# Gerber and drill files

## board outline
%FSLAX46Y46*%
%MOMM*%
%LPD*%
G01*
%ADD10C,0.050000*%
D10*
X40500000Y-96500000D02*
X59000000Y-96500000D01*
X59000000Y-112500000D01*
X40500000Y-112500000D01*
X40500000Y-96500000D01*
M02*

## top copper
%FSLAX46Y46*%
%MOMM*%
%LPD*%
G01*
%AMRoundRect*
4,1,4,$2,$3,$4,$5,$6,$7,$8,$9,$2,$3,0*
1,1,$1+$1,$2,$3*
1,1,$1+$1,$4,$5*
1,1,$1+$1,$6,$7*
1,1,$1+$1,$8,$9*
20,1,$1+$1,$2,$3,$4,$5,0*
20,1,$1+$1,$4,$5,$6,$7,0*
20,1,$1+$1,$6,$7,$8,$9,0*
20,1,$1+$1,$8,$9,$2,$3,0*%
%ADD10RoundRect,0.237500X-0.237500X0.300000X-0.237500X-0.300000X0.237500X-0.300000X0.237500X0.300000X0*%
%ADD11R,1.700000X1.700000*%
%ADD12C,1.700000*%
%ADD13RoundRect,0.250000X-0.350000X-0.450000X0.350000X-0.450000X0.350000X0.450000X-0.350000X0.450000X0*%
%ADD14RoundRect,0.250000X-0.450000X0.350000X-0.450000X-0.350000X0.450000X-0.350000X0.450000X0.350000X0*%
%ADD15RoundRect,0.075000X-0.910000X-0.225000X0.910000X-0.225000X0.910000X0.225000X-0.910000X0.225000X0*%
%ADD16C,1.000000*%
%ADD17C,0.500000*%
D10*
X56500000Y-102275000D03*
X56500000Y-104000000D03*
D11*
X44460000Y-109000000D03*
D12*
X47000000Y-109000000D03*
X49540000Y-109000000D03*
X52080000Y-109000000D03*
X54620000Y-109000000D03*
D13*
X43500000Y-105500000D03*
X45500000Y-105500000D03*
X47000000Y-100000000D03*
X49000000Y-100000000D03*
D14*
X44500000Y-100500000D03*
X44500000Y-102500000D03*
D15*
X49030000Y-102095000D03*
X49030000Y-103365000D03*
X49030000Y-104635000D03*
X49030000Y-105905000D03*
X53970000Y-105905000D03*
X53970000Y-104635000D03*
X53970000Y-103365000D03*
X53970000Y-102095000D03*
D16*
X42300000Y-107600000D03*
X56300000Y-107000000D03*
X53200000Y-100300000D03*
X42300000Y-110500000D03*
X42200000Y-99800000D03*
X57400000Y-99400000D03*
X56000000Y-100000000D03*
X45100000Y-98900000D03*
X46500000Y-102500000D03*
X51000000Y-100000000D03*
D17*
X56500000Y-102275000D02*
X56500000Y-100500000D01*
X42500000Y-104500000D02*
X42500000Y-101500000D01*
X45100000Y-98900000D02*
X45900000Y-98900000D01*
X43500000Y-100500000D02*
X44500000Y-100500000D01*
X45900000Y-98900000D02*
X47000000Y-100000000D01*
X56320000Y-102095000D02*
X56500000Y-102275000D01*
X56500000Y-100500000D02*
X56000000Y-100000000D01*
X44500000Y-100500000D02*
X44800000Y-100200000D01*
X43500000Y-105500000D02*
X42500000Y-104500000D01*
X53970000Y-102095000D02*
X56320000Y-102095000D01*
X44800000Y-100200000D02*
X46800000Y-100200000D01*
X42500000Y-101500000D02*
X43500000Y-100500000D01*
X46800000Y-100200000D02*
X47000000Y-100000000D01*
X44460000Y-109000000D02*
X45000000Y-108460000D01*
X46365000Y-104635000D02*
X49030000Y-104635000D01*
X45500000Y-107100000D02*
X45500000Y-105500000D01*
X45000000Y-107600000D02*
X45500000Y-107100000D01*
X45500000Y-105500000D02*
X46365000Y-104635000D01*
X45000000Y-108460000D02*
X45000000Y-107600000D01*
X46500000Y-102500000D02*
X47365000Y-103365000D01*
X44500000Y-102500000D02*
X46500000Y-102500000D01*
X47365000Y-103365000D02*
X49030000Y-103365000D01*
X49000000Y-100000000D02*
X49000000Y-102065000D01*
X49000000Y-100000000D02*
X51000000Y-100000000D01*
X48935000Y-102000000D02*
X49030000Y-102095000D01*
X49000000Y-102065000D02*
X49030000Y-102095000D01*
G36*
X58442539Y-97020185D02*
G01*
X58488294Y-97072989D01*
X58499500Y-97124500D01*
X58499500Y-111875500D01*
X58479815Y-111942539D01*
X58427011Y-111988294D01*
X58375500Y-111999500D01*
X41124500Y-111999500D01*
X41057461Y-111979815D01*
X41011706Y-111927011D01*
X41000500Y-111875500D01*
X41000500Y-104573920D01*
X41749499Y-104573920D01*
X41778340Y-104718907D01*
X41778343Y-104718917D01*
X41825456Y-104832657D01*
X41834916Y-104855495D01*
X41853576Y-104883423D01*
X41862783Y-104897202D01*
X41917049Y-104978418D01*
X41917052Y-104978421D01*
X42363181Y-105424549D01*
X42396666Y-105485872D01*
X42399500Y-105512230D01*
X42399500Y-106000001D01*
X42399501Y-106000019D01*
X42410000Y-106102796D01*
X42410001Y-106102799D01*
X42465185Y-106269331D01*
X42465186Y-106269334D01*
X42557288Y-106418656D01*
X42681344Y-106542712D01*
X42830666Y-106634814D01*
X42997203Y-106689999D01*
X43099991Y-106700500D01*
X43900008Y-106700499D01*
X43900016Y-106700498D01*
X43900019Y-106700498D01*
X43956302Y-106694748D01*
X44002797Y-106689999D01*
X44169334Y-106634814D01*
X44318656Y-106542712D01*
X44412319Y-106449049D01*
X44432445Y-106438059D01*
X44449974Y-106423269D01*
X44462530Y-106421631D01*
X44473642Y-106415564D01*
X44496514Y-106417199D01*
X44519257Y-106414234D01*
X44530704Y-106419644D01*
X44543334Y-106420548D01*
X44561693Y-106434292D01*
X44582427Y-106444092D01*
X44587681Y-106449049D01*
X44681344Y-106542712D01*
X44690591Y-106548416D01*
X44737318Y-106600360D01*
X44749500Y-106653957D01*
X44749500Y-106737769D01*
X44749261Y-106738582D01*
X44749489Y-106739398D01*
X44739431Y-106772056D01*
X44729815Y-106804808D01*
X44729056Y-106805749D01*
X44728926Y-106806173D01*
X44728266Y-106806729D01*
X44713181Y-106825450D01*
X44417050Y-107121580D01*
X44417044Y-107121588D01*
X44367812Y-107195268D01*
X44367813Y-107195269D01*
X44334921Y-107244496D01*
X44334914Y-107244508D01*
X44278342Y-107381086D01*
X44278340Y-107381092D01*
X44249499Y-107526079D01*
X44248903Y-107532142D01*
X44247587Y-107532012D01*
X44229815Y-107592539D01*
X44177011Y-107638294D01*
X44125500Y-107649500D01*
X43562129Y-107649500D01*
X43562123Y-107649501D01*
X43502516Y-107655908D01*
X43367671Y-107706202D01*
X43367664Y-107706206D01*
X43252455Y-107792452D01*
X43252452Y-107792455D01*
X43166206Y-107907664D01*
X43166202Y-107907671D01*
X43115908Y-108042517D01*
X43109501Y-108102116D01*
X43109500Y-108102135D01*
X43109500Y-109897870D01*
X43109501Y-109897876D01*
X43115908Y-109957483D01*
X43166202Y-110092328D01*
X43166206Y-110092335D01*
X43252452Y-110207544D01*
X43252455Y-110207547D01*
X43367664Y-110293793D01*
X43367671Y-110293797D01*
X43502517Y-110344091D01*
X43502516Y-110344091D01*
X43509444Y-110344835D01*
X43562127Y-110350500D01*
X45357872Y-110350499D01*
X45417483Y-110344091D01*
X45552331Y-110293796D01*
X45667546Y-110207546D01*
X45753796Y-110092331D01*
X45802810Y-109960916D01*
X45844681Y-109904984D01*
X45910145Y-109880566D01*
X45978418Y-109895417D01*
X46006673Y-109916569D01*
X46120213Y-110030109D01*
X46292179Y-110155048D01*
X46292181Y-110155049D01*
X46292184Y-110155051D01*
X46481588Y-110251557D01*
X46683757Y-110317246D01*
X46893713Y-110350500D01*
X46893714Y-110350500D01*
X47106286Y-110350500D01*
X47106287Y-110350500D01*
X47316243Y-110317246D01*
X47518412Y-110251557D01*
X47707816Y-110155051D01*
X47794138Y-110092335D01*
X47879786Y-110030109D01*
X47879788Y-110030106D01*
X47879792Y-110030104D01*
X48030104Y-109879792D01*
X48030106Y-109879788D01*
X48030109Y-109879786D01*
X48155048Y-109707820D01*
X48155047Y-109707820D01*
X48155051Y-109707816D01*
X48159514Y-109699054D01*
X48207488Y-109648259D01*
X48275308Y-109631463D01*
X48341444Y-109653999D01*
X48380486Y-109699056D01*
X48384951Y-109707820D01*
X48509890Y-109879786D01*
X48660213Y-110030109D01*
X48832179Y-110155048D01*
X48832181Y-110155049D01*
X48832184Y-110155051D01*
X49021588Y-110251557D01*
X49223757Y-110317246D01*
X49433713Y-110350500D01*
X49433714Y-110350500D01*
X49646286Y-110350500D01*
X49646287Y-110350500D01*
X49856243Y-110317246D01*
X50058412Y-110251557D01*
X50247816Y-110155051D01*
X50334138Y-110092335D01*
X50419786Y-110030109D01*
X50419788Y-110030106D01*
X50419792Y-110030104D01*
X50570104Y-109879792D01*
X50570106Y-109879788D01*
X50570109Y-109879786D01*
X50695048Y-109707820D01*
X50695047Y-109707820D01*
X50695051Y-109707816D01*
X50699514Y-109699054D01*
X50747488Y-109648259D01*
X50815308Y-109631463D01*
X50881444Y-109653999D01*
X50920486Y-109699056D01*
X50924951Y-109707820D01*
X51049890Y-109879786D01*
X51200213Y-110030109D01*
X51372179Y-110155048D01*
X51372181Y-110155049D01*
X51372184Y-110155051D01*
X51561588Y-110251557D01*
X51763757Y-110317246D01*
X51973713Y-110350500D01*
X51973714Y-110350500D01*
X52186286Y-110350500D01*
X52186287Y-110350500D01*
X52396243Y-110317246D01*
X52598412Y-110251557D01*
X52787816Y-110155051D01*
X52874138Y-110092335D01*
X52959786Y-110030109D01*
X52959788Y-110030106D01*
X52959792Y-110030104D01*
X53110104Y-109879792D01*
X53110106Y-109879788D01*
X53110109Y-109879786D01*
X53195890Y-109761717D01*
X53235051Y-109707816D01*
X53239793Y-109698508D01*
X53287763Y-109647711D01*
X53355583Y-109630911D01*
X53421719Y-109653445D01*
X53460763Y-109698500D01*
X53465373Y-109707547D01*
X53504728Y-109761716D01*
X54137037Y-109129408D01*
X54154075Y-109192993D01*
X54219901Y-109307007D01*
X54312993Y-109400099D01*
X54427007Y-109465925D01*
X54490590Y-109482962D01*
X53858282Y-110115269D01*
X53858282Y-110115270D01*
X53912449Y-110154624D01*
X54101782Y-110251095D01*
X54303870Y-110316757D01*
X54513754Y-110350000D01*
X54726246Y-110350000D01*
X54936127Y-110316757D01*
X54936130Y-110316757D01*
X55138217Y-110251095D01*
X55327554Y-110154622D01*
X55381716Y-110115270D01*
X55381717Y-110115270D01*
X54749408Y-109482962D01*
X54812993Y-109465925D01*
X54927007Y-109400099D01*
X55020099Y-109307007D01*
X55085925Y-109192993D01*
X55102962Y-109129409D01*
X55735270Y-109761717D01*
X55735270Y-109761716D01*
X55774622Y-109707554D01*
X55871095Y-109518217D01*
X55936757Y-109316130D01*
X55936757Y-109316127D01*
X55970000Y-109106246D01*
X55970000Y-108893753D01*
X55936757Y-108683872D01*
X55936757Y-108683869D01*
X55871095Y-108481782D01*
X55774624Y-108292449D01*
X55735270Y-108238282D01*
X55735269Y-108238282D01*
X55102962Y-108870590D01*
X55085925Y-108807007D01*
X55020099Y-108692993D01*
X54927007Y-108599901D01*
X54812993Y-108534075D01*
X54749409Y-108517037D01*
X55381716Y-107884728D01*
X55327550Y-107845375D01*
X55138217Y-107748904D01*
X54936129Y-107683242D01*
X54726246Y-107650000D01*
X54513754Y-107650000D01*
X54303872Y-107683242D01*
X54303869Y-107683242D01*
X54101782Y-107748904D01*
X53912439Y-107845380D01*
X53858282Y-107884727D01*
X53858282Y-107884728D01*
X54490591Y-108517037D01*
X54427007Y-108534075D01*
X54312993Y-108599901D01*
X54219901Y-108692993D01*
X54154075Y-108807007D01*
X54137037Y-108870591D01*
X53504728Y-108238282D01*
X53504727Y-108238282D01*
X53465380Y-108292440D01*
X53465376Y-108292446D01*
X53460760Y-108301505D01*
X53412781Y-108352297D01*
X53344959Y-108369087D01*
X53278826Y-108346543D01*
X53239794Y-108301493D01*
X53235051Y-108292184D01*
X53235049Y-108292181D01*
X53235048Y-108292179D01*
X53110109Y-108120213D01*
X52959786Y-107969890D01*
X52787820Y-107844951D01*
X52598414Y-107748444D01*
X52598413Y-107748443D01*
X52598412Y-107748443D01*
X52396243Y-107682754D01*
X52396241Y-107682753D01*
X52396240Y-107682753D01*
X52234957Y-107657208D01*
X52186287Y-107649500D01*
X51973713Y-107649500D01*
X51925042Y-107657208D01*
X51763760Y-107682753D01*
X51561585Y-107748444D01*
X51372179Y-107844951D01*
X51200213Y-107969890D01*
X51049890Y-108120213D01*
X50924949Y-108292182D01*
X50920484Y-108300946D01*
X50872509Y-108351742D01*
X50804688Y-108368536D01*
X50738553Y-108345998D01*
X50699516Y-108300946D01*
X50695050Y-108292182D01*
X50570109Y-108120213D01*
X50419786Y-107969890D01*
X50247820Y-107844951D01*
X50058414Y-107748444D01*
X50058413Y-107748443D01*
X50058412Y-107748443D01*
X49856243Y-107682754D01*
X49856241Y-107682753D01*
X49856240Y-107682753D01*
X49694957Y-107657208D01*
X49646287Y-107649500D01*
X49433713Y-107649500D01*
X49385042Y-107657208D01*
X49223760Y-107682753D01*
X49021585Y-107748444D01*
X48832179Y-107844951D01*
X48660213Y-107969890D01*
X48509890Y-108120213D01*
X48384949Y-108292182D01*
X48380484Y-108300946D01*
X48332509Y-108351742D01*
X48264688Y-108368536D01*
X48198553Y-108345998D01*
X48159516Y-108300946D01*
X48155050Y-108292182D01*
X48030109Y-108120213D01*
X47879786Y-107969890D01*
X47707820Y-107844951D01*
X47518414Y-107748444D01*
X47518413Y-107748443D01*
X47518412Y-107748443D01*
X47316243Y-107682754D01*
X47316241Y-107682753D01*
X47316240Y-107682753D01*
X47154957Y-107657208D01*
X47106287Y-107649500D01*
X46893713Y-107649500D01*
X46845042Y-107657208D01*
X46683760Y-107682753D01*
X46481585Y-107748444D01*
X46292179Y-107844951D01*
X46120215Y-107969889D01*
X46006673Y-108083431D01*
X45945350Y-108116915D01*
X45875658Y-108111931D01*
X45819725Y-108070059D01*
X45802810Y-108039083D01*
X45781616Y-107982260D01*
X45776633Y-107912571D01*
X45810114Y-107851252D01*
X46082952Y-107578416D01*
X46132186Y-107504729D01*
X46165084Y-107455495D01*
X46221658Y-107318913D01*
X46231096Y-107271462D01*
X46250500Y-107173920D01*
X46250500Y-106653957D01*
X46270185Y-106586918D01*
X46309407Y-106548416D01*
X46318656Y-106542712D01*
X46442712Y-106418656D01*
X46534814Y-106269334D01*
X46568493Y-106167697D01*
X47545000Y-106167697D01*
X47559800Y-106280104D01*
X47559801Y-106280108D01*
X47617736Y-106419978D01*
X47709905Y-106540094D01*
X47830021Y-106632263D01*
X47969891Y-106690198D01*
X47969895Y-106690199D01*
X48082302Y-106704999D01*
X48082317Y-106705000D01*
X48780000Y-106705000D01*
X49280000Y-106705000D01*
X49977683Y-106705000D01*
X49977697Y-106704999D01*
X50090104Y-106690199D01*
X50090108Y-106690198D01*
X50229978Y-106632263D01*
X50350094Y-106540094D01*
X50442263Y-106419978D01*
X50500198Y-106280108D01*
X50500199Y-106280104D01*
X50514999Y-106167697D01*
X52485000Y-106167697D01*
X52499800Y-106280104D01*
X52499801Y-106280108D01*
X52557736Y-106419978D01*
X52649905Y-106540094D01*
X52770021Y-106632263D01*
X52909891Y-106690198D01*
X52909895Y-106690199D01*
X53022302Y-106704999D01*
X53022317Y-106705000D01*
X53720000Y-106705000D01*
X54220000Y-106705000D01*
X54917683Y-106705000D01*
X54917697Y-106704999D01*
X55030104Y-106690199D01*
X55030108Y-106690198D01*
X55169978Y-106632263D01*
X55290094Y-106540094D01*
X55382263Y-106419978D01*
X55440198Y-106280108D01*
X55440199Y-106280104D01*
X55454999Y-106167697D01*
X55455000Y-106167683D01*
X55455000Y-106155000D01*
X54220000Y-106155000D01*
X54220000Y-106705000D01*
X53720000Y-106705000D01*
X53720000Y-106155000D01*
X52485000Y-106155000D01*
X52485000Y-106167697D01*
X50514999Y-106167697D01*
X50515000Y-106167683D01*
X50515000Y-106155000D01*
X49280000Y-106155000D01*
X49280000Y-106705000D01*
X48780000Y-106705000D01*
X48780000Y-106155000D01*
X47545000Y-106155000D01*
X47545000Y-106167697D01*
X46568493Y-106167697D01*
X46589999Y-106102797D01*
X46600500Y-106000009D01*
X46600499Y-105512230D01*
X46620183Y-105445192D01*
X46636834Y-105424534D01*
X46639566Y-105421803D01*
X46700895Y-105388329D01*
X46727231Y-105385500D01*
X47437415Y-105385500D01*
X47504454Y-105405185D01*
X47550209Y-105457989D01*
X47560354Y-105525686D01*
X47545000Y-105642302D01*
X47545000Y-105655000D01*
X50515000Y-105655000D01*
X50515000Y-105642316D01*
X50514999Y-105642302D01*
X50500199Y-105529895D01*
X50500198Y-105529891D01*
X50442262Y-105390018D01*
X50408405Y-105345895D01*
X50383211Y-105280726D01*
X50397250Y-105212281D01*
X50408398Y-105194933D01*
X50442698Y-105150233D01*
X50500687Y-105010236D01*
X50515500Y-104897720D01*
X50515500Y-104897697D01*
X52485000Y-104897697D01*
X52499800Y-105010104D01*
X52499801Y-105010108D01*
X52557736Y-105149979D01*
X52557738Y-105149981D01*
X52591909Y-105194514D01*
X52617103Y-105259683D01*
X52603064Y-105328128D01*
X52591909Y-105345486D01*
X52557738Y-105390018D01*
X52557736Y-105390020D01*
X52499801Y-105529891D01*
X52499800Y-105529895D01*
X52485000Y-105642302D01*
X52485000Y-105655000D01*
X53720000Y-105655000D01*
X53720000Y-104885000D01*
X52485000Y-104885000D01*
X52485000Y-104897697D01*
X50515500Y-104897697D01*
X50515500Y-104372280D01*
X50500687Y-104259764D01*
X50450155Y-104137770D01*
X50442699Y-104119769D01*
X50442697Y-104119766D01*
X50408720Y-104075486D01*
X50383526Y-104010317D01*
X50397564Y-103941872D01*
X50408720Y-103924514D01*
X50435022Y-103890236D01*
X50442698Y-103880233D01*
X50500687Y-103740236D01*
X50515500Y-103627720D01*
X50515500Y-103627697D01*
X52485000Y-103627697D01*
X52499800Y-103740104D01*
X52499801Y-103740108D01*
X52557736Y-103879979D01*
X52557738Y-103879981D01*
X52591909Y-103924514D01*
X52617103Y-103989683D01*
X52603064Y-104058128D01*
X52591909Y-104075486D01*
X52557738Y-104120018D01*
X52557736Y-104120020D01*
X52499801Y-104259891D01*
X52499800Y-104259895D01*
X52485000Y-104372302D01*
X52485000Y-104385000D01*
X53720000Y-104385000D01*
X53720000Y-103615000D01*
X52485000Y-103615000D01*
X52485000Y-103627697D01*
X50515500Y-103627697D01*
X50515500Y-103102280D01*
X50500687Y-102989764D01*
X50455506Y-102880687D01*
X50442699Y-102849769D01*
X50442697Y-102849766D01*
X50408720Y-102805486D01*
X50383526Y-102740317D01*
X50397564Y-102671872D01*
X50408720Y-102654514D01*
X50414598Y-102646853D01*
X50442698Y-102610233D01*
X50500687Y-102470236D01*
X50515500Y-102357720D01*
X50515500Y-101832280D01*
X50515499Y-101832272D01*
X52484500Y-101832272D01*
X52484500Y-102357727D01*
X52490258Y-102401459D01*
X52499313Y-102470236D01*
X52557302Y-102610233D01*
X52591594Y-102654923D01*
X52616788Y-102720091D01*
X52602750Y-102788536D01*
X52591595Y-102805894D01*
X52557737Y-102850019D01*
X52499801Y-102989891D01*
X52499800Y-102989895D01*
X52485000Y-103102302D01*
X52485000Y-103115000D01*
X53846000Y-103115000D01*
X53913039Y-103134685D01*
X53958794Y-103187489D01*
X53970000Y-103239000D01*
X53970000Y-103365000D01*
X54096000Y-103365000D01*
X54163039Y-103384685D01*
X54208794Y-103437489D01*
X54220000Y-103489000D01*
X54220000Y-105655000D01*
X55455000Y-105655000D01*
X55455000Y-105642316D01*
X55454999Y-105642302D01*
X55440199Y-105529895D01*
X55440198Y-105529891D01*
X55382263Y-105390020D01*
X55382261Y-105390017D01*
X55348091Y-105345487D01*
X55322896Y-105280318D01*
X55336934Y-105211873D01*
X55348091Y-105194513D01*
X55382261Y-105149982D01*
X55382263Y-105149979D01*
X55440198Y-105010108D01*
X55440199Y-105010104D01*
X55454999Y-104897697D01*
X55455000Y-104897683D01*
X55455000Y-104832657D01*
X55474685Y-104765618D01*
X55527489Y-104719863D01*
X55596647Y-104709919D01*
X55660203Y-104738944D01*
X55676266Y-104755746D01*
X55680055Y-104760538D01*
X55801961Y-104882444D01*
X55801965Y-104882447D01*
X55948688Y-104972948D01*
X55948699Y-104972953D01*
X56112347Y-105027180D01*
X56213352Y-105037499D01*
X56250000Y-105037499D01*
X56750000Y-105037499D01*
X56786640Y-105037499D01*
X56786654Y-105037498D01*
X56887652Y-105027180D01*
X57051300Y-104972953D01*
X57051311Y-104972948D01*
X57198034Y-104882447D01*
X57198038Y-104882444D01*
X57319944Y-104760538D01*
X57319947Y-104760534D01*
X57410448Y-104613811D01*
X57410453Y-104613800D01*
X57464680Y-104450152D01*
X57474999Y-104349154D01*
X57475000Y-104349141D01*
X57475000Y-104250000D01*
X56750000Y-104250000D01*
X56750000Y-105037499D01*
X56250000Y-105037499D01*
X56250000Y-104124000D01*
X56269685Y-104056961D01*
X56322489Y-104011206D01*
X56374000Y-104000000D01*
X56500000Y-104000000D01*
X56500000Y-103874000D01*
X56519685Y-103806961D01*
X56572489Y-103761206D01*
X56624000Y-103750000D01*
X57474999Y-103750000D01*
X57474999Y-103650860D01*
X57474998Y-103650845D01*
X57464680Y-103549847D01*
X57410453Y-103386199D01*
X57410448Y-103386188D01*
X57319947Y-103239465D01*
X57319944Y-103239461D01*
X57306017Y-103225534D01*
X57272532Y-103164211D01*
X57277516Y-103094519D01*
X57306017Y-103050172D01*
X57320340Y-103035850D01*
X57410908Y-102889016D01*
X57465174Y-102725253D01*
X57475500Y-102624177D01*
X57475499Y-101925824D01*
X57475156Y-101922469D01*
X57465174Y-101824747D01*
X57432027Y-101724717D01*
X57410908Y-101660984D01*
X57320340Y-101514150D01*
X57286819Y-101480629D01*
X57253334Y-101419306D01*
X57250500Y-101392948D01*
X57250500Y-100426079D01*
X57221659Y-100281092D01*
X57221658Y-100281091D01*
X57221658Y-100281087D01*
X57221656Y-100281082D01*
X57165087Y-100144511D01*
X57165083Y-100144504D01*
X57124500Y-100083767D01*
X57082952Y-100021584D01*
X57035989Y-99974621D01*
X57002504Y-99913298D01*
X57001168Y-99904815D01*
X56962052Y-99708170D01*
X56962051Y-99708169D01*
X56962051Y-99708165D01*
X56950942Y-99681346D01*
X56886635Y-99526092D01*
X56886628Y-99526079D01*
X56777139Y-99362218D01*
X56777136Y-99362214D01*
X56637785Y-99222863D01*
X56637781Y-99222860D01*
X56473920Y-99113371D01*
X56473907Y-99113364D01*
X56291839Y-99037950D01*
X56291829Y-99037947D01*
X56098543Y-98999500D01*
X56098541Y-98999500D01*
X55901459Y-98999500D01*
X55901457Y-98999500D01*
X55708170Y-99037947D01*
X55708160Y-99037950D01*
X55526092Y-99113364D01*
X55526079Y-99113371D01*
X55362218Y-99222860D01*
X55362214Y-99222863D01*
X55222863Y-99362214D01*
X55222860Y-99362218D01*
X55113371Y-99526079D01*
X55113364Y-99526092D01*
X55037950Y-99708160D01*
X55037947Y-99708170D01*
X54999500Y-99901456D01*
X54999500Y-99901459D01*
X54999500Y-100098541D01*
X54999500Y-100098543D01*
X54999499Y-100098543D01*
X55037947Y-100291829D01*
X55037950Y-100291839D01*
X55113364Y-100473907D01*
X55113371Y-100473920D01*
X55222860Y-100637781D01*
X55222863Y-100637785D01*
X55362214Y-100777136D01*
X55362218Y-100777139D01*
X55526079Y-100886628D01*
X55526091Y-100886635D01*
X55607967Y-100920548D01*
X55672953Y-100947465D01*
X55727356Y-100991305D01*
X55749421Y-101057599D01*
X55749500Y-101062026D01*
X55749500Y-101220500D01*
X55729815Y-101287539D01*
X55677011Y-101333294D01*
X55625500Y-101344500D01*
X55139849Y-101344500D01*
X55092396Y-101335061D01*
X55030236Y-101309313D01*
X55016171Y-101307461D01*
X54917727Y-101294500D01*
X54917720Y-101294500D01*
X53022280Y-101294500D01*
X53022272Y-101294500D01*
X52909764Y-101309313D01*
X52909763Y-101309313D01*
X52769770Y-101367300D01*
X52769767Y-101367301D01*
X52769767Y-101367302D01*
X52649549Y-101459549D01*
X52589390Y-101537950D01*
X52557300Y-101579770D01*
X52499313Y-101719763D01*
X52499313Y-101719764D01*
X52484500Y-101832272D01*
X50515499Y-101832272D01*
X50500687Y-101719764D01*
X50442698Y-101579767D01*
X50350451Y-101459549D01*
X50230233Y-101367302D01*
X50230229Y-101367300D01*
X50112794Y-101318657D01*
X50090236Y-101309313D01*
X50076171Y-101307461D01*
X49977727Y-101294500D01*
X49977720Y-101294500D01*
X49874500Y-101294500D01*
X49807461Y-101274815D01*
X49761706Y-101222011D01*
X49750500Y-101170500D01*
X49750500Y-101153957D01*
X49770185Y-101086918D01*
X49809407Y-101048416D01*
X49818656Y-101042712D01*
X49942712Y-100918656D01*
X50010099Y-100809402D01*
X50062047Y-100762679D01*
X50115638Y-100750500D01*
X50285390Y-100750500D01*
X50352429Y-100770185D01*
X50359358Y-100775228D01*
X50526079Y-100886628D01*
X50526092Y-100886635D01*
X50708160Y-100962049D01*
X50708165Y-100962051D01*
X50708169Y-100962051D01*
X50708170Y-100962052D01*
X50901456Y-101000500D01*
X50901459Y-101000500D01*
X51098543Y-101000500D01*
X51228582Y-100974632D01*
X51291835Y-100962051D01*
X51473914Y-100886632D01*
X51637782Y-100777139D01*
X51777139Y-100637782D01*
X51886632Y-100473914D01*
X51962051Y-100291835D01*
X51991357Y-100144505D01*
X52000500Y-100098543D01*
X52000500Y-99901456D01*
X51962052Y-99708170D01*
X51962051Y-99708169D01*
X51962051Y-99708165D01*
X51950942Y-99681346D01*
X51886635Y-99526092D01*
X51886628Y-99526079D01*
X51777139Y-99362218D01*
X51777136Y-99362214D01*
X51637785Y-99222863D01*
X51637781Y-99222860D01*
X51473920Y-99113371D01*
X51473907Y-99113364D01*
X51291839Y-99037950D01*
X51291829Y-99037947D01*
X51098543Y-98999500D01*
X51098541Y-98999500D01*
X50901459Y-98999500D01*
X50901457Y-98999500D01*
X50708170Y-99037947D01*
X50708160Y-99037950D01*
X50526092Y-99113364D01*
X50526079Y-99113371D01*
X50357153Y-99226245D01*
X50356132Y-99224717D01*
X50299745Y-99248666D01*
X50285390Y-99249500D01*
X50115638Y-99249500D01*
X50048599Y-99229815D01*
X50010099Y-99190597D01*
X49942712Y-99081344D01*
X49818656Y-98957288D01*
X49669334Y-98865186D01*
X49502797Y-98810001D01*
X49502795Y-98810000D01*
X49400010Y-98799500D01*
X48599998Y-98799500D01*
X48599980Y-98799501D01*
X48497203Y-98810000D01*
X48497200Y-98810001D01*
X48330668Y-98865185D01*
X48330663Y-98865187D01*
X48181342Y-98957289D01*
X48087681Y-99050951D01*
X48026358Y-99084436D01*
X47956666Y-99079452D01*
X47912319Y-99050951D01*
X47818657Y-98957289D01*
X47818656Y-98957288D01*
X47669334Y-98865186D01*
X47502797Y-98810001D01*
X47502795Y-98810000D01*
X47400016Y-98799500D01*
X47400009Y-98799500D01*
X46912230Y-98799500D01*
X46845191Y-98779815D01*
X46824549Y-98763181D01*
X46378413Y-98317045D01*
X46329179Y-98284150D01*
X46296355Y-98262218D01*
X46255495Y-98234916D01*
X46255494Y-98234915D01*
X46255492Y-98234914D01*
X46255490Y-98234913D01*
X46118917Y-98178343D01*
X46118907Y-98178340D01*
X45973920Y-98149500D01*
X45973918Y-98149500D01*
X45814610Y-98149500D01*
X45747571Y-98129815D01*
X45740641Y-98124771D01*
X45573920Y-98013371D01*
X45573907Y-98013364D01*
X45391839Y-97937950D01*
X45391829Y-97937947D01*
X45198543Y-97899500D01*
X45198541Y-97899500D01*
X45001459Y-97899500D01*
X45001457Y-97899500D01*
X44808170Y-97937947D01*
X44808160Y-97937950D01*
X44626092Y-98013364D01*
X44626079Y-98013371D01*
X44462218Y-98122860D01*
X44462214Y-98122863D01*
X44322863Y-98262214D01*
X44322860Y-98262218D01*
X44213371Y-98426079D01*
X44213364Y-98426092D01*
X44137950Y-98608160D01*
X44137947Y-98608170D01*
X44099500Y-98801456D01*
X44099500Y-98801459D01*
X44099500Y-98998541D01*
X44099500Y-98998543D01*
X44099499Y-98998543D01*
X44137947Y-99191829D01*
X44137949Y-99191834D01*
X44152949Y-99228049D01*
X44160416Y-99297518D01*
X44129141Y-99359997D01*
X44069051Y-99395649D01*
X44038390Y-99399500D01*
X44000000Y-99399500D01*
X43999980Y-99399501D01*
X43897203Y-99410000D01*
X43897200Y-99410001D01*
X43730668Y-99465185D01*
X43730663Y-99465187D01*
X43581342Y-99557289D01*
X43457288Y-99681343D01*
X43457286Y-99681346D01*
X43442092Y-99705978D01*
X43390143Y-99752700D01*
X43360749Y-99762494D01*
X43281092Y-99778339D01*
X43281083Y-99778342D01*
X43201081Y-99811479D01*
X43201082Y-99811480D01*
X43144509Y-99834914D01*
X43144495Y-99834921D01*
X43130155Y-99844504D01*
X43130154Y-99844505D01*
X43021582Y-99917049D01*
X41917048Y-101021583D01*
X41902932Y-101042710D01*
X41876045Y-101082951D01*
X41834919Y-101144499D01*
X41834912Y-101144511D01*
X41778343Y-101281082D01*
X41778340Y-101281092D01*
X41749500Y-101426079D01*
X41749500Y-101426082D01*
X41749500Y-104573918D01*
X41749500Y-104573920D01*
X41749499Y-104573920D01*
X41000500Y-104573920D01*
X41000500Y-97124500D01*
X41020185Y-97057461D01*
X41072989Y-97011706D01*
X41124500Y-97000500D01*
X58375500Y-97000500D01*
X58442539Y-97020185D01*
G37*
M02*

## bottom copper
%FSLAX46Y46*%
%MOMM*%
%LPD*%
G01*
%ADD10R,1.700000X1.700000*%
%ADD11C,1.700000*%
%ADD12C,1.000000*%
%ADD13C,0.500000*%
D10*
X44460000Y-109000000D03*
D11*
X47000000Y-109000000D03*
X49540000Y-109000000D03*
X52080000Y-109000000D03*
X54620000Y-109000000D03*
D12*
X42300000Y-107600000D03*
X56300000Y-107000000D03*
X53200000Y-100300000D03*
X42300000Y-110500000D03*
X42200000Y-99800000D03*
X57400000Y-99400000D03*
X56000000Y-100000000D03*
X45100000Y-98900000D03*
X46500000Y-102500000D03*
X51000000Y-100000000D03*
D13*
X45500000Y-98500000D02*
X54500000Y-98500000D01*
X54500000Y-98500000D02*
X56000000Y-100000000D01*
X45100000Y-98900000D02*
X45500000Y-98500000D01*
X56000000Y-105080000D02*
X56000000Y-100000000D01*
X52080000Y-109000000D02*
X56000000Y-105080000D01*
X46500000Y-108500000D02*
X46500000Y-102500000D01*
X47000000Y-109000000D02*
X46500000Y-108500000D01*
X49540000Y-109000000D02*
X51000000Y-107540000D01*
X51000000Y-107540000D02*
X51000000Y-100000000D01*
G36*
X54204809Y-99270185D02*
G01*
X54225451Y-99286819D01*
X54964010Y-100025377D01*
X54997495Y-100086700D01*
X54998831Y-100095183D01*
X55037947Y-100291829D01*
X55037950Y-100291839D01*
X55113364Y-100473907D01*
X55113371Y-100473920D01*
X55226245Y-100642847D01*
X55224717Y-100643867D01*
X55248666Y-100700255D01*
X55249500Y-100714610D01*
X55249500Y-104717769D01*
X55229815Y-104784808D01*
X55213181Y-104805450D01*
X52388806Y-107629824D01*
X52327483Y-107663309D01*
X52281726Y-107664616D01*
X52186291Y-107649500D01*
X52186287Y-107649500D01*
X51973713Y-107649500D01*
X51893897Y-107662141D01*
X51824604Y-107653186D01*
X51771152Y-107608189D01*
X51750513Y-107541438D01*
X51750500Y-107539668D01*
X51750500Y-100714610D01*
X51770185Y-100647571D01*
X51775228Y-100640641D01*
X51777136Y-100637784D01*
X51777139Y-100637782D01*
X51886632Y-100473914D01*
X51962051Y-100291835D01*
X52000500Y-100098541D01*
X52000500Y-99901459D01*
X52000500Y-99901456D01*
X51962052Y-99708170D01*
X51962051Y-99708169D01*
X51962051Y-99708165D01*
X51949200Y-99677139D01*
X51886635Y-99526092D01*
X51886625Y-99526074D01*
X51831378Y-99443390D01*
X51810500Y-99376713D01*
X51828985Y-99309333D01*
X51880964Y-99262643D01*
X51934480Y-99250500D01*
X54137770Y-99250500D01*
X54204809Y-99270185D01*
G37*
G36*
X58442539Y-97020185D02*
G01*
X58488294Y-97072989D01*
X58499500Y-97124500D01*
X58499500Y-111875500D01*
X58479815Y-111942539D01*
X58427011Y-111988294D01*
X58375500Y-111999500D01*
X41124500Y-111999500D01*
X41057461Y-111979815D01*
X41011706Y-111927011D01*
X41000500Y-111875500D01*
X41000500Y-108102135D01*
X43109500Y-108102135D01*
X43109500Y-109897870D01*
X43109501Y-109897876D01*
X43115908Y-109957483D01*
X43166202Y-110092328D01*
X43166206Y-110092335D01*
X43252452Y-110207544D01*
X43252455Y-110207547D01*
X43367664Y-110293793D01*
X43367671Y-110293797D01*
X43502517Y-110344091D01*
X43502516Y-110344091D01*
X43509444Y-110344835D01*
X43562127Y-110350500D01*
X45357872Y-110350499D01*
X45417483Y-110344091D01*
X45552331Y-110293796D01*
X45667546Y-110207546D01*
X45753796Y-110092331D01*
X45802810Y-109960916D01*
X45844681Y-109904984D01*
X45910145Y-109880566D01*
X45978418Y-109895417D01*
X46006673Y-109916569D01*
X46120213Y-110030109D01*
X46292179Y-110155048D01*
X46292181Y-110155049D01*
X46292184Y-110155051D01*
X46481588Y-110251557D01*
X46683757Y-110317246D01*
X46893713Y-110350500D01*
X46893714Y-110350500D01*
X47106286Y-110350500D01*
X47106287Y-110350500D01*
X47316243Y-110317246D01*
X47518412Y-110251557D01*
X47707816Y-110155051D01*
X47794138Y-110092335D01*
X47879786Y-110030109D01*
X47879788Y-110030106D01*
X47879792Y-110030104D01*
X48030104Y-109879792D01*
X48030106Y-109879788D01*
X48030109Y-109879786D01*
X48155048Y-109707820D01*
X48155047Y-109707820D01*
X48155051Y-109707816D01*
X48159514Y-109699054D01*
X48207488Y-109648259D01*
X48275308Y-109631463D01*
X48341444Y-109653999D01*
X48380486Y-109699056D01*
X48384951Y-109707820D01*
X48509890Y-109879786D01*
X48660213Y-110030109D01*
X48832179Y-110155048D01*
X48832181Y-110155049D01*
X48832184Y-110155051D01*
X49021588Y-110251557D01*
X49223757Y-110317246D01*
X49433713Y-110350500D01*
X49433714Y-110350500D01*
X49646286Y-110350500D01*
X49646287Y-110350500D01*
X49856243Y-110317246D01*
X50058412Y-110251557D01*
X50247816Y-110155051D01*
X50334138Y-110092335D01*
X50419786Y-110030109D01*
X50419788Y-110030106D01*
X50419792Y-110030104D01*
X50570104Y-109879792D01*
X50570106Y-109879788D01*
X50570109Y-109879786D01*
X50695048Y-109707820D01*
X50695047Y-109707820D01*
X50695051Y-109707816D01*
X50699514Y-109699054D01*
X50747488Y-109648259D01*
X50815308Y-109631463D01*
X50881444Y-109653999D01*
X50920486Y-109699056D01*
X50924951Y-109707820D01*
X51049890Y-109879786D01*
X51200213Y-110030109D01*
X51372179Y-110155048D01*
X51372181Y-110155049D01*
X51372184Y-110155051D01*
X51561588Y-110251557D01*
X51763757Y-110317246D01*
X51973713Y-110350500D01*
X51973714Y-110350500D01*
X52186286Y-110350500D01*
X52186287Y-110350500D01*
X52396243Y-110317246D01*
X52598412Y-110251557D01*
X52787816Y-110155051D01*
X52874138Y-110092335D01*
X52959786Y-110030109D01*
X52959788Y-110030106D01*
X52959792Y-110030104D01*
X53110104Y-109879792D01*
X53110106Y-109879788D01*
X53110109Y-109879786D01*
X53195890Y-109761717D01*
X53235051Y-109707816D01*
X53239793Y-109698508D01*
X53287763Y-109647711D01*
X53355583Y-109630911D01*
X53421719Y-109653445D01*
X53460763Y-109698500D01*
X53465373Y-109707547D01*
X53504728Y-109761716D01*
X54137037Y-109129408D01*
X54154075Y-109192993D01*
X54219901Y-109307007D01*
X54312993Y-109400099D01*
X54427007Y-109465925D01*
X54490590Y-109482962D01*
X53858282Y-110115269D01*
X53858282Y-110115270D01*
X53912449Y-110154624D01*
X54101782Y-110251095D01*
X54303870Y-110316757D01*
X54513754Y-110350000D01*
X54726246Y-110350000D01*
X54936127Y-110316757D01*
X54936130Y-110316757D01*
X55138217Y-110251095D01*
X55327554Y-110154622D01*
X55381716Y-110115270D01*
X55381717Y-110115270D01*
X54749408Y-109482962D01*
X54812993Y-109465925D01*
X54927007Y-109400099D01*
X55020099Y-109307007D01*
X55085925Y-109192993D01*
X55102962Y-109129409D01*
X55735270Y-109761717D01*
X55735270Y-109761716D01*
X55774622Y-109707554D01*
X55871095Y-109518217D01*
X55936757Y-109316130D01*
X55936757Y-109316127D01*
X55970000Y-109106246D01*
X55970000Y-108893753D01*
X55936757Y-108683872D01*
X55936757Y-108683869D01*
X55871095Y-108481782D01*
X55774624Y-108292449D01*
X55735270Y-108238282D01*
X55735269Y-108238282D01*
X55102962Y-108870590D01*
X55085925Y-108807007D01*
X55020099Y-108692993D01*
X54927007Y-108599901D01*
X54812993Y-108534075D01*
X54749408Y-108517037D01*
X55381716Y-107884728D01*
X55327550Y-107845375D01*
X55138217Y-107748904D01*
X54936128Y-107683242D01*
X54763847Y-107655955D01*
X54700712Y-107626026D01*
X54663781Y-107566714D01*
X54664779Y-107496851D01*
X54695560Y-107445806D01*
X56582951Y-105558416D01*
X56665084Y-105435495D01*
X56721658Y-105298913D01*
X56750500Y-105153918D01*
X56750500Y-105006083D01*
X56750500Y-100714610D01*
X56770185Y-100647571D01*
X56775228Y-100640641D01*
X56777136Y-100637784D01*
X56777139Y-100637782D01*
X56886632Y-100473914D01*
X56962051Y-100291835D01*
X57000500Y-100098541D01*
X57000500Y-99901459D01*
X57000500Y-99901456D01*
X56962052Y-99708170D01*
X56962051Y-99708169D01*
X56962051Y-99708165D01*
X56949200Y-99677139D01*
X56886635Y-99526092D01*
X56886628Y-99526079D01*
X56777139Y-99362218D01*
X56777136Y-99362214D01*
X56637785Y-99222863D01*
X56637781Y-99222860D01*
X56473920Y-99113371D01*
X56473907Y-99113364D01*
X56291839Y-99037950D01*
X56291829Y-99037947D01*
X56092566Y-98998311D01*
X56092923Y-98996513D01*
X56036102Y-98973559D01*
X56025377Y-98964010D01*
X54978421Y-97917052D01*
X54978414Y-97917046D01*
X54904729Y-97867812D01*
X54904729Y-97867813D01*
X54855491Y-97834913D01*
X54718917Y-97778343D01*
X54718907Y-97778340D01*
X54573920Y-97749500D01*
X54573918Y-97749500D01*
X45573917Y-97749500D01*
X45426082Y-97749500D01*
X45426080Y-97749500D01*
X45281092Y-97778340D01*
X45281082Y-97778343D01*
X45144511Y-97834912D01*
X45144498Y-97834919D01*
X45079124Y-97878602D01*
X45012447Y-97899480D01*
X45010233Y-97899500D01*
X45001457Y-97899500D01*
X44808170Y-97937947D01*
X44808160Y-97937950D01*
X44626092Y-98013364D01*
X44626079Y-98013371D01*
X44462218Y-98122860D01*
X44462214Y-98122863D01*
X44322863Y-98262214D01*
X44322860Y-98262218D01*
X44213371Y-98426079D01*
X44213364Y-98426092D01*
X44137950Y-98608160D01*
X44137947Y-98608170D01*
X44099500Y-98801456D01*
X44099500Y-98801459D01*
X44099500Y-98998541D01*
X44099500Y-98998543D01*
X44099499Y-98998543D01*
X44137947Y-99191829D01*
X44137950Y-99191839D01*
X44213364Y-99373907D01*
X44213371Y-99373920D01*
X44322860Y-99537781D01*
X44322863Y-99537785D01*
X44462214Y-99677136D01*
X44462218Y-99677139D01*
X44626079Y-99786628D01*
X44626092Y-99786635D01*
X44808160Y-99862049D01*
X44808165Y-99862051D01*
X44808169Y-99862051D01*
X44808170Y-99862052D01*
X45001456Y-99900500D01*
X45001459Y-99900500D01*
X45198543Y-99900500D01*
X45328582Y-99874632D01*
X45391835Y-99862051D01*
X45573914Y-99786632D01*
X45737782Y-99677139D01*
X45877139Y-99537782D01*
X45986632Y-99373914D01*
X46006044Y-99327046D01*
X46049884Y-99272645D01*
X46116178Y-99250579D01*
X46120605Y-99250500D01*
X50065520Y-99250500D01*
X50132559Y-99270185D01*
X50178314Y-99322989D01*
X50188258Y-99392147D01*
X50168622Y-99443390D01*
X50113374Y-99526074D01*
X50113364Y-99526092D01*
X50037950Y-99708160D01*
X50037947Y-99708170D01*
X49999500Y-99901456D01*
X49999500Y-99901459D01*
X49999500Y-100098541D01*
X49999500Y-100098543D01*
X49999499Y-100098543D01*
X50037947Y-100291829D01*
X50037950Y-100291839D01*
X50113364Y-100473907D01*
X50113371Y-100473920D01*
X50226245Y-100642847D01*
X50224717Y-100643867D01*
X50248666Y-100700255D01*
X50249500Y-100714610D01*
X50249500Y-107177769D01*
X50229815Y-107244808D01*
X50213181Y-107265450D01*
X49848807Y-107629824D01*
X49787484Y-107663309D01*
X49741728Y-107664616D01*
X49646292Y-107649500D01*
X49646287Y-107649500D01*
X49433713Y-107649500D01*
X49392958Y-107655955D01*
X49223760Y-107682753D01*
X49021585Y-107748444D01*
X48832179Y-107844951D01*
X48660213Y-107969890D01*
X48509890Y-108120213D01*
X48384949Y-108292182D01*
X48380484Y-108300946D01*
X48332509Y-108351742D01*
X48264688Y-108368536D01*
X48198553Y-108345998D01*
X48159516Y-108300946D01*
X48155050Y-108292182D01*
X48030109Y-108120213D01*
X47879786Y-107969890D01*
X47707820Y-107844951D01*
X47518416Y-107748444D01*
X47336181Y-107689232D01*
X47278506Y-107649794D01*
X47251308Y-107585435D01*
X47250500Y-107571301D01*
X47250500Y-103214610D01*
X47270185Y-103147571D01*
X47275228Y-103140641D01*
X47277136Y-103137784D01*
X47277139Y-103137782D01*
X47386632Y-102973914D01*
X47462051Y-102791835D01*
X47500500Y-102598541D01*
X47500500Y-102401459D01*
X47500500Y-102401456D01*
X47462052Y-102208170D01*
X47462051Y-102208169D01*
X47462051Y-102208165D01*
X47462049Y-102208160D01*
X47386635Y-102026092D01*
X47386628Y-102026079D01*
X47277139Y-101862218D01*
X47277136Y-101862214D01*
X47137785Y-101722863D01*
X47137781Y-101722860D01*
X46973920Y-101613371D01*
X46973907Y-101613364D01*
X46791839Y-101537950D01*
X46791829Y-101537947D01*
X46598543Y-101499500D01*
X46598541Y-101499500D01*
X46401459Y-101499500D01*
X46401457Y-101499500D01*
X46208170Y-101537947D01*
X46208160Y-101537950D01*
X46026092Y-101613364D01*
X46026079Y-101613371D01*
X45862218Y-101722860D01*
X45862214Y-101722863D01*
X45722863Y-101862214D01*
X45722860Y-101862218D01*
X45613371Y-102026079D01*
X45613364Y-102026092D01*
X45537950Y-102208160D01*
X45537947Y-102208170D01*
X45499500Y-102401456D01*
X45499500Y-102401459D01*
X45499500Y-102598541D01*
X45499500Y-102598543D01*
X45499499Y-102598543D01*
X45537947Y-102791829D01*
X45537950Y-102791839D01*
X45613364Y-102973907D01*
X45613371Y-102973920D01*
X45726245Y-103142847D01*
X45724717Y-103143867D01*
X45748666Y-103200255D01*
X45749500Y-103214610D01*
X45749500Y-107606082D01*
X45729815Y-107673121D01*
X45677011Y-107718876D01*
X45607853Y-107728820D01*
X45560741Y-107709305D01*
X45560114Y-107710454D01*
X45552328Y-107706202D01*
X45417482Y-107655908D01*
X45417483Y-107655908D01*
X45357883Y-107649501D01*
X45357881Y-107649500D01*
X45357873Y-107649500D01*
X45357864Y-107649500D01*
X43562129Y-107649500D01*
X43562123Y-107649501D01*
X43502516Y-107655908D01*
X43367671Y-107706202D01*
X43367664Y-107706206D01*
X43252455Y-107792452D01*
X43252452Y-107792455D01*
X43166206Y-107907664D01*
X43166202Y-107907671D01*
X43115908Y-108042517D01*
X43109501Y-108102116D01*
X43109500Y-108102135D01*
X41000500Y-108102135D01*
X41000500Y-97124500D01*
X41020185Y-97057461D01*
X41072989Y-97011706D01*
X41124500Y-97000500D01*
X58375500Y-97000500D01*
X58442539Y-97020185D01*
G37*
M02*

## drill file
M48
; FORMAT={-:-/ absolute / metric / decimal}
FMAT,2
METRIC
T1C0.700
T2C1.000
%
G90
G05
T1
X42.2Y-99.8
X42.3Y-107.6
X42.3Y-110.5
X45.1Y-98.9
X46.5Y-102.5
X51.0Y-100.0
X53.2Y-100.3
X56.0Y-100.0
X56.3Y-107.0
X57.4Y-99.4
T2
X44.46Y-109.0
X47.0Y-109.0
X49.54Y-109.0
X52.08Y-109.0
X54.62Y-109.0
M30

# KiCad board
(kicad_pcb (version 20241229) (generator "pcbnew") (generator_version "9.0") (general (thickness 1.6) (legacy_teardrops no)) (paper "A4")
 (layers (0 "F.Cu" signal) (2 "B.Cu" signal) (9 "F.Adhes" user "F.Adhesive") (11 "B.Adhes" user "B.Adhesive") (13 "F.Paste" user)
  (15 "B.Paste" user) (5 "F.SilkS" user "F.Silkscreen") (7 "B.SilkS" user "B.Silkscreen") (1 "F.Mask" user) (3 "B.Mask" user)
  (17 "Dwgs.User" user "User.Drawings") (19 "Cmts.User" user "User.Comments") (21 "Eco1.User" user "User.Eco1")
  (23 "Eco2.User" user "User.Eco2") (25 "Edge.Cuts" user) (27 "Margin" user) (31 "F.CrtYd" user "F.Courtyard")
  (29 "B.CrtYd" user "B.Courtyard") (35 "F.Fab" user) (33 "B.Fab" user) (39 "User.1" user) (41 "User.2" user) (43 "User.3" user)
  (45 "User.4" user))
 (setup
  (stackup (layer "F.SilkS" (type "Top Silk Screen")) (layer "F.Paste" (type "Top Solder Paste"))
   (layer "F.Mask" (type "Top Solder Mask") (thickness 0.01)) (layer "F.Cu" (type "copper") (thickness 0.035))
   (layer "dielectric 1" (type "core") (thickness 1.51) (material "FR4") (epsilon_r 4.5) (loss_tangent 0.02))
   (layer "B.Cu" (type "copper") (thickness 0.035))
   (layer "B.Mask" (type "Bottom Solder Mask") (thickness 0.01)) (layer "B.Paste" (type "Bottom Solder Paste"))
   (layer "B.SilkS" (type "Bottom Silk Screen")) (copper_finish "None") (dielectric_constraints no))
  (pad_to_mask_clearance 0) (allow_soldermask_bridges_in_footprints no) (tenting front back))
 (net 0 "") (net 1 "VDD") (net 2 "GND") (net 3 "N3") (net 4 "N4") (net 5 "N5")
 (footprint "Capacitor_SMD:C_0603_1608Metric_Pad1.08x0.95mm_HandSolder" (layer "F.Cu") (at 56.5 103.1375 -90)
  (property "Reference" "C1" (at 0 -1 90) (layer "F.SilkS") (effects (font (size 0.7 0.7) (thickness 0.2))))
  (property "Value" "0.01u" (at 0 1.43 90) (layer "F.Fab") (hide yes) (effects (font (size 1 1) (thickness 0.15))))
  (pad "1" smd roundrect (at -0.8625 0 270) (size 1.075 0.95) (layers "F.Cu" "F.Mask" "F.Paste") (roundrect_rratio 0.25) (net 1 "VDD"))
  (pad "2" smd roundrect (at 0.8625 0 270) (size 1.075 0.95) (layers "F.Cu" "F.Mask" "F.Paste") (roundrect_rratio 0.25) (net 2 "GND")))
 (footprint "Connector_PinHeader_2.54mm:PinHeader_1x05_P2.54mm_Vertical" (layer "F.Cu") (at 44.46 109 90)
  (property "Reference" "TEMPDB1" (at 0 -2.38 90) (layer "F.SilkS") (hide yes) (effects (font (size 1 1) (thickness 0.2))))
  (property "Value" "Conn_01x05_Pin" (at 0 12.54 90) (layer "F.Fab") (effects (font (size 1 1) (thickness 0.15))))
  (pad "1" thru_hole rect (at 0 0 90) (size 1.7 1.7) (drill 1) (layers "*.Cu" "*.Mask") (remove_unused_layers no) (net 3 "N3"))
  (pad "2" thru_hole circle (at 0 2.54 90) (size 1.7 1.7) (drill 1) (layers "*.Cu" "*.Mask") (remove_unused_layers no) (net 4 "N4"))
  (pad "3" thru_hole circle (at 0 5.08 90) (size 1.7 1.7) (drill 1) (layers "*.Cu" "*.Mask") (remove_unused_layers no) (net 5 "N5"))
  (pad "4" thru_hole circle (at 0 7.62 90) (size 1.7 1.7) (drill 1) (layers "*.Cu" "*.Mask") (remove_unused_layers no) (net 1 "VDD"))
  (pad "5" thru_hole circle (at 0 10.16 90) (size 1.7 1.7) (drill 1) (layers "*.Cu" "*.Mask") (remove_unused_layers no) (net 2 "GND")))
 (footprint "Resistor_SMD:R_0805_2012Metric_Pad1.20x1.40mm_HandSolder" (layer "F.Cu") (at 44.5 105.5)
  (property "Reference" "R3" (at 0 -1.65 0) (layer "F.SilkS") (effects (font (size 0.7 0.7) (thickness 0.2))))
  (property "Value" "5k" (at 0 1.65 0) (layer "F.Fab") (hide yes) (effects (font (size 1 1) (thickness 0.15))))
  (pad "1" smd roundrect (at -1 0) (size 1.2 1.4) (layers "F.Cu" "F.Mask" "F.Paste") (roundrect_rratio 0.208333) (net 1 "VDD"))
  (pad "2" smd roundrect (at 1 0) (size 1.2 1.4) (layers "F.Cu" "F.Mask" "F.Paste") (roundrect_rratio 0.208333) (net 3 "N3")))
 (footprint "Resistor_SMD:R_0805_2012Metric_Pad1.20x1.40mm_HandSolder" (layer "F.Cu") (at 48 100)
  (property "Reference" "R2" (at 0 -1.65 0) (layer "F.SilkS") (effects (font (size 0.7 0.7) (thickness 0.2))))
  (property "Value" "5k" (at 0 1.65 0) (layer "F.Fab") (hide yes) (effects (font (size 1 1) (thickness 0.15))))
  (pad "1" smd roundrect (at -1 0) (size 1.2 1.4) (layers "F.Cu" "F.Mask" "F.Paste") (roundrect_rratio 0.208333) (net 1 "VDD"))
  (pad "2" smd roundrect (at 1 0) (size 1.2 1.4) (layers "F.Cu" "F.Mask" "F.Paste") (roundrect_rratio 0.208333) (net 5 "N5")))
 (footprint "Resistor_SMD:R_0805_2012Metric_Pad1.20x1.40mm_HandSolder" (layer "F.Cu") (at 44.5 101.5 -90)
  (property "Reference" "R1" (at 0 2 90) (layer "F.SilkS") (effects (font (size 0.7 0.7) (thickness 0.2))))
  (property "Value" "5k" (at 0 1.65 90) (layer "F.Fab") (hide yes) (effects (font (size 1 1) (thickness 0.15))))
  (pad "1" smd roundrect (at -1 0 270) (size 1.2 1.4) (layers "F.Cu" "F.Mask" "F.Paste") (roundrect_rratio 0.208333) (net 1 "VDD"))
  (pad "2" smd roundrect (at 1 0 270) (size 1.2 1.4) (layers "F.Cu" "F.Mask" "F.Paste") (roundrect_rratio 0.208333) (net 4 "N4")))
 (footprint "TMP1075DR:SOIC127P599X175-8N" (layer "F.Cu") (at 51.5 104)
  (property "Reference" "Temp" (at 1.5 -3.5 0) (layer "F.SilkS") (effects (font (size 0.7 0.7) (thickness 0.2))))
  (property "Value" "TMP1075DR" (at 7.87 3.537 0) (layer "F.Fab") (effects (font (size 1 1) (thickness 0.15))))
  (pad "1" smd roundrect (at -2.47 -1.905) (size 1.97 0.6) (layers "F.Cu" "F.Mask" "F.Paste") (roundrect_rratio 0.125) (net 5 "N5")
   (solder_mask_margin 0.102))
  (pad "2" smd roundrect (at -2.47 -0.635) (size 1.97 0.6) (layers "F.Cu" "F.Mask" "F.Paste") (roundrect_rratio 0.125) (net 4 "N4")
   (solder_mask_margin 0.102))
  (pad "3" smd roundrect (at -2.47 0.635) (size 1.97 0.6) (layers "F.Cu" "F.Mask" "F.Paste") (roundrect_rratio 0.125) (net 3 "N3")
   (solder_mask_margin 0.102))
  (pad "4" smd roundrect (at -2.47 1.905) (size 1.97 0.6) (layers "F.Cu" "F.Mask" "F.Paste") (roundrect_rratio 0.125) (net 2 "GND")
   (solder_mask_margin 0.102))
  (pad "5" smd roundrect (at 2.47 1.905) (size 1.97 0.6) (layers "F.Cu" "F.Mask" "F.Paste") (roundrect_rratio 0.125) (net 2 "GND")
   (solder_mask_margin 0.102))
  (pad "6" smd roundrect (at 2.47 0.635) (size 1.97 0.6) (layers "F.Cu" "F.Mask" "F.Paste") (roundrect_rratio 0.125) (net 2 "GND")
   (solder_mask_margin 0.102))
  (pad "7" smd roundrect (at 2.47 -0.635) (size 1.97 0.6) (layers "F.Cu" "F.Mask" "F.Paste") (roundrect_rratio 0.125) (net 2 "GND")
   (solder_mask_margin 0.102))
  (pad "8" smd roundrect (at 2.47 -1.905) (size 1.97 0.6) (layers "F.Cu" "F.Mask" "F.Paste") (roundrect_rratio 0.125) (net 1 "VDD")
   (solder_mask_margin 0.102)))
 (gr_rect (start 40.5 96.5) (end 59 112.5) (stroke (width 0.05) (type default)) (fill no) (layer "Edge.Cuts"))
 (via (at 42.3 107.6) (size 1) (drill 0.7) (layers "F.Cu" "B.Cu") (free yes) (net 2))
 (via (at 56.3 107) (size 1) (drill 0.7) (layers "F.Cu" "B.Cu") (free yes) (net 2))
 (via (at 53.2 100.3) (size 1) (drill 0.7) (layers "F.Cu" "B.Cu") (free yes) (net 2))
 (via (at 42.3 110.5) (size 1) (drill 0.7) (layers "F.Cu" "B.Cu") (free yes) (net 2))
 (via (at 42.2 99.8) (size 1) (drill 0.7) (layers "F.Cu" "B.Cu") (free yes) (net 2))
 (via (at 57.4 99.4) (size 1) (drill 0.7) (layers "F.Cu" "B.Cu") (free yes) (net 2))
 (segment (start 56.5 102.275) (end 56.5 100.5) (width 0.5) (layer "F.Cu") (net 1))
 (segment (start 42.5 104.5) (end 42.5 101.5) (width 0.5) (layer "F.Cu") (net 1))
 (segment (start 45.1 98.9) (end 45.9 98.9) (width 0.5) (layer "F.Cu") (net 1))
 (segment (start 43.5 100.5) (end 44.5 100.5) (width 0.5) (layer "F.Cu") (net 1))
 (segment (start 45.9 98.9) (end 47 100) (width 0.5) (layer "F.Cu") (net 1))
 (segment (start 56.32 102.095) (end 56.5 102.275) (width 0.5) (layer "F.Cu") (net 1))
 (segment (start 56.5 100.5) (end 56 100) (width 0.5) (layer "F.Cu") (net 1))
 (segment (start 44.5 100.5) (end 44.8 100.2) (width 0.5) (layer "F.Cu") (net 1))
 (segment (start 43.5 105.5) (end 42.5 104.5) (width 0.5) (layer "F.Cu") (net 1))
 (segment (start 53.97 102.095) (end 56.32 102.095) (width 0.5) (layer "F.Cu") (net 1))
 (segment (start 44.8 100.2) (end 46.8 100.2) (width 0.5) (layer "F.Cu") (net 1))
 (segment (start 42.5 101.5) (end 43.5 100.5) (width 0.5) (layer "F.Cu") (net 1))
 (segment (start 46.8 100.2) (end 47 100) (width 0.5) (layer "F.Cu") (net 1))
 (via (at 56 100) (size 1) (drill 0.7) (layers "F.Cu" "B.Cu") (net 1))
 (via (at 45.1 98.9) (size 1) (drill 0.7) (layers "F.Cu" "B.Cu") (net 1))
 (segment (start 45.5 98.5) (end 54.5 98.5) (width 0.5) (layer "B.Cu") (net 1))
 (segment (start 54.5 98.5) (end 56 100) (width 0.5) (layer "B.Cu") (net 1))
 (segment (start 45.1 98.9) (end 45.5 98.5) (width 0.5) (layer "B.Cu") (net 1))
 (segment (start 56 105.08) (end 56 100) (width 0.5) (layer "B.Cu") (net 1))
 (segment (start 52.08 109) (end 56 105.08) (width 0.5) (layer "B.Cu") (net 1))
 (segment (start 44.46 109) (end 45 108.46) (width 0.5) (layer "F.Cu") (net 3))
 (segment (start 46.365 104.635) (end 49.03 104.635) (width 0.5) (layer "F.Cu") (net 3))
 (segment (start 45.5 107.1) (end 45.5 105.5) (width 0.5) (layer "F.Cu") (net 3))
 (segment (start 45 107.6) (end 45.5 107.1) (width 0.5) (layer "F.Cu") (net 3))
 (segment (start 45.5 105.5) (end 46.365 104.635) (width 0.5) (layer "F.Cu") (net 3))
 (segment (start 45 108.46) (end 45 107.6) (width 0.5) (layer "F.Cu") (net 3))
 (segment (start 46.5 102.5) (end 47.365 103.365) (width 0.5) (layer "F.Cu") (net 4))
 (segment (start 44.5 102.5) (end 46.5 102.5) (width 0.5) (layer "F.Cu") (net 4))
 (segment (start 47.365 103.365) (end 49.03 103.365) (width 0.5) (layer "F.Cu") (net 4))
 (via (at 46.5 102.5) (size 1) (drill 0.7) (layers "F.Cu" "B.Cu") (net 4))
 (segment (start 46.5 108.5) (end 46.5 102.5) (width 0.5) (layer "B.Cu") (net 4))
 (segment (start 47 109) (end 46.5 108.5) (width 0.5) (layer "B.Cu") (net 4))
 (segment (start 49 100) (end 49 102.065) (width 0.5) (layer "F.Cu") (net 5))
 (segment (start 49 100) (end 51 100) (width 0.5) (layer "F.Cu") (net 5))
 (segment (start 48.935 102) (end 49.03 102.095) (width 0.5) (layer "F.Cu") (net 5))
 (segment (start 49 102.065) (end 49.03 102.095) (width 0.5) (layer "F.Cu") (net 5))
 (via (at 51 100) (size 1) (drill 0.7) (layers "F.Cu" "B.Cu") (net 5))
 (segment (start 49.54 109) (end 51 107.54) (width 0.5) (layer "B.Cu") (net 5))
 (segment (start 51 107.54) (end 51 100) (width 0.5) (layer "B.Cu") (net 5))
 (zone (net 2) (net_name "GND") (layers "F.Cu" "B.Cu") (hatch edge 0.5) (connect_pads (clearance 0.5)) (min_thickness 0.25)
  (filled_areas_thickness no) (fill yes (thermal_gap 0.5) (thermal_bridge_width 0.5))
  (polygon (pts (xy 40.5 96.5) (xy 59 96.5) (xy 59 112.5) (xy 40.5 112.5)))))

